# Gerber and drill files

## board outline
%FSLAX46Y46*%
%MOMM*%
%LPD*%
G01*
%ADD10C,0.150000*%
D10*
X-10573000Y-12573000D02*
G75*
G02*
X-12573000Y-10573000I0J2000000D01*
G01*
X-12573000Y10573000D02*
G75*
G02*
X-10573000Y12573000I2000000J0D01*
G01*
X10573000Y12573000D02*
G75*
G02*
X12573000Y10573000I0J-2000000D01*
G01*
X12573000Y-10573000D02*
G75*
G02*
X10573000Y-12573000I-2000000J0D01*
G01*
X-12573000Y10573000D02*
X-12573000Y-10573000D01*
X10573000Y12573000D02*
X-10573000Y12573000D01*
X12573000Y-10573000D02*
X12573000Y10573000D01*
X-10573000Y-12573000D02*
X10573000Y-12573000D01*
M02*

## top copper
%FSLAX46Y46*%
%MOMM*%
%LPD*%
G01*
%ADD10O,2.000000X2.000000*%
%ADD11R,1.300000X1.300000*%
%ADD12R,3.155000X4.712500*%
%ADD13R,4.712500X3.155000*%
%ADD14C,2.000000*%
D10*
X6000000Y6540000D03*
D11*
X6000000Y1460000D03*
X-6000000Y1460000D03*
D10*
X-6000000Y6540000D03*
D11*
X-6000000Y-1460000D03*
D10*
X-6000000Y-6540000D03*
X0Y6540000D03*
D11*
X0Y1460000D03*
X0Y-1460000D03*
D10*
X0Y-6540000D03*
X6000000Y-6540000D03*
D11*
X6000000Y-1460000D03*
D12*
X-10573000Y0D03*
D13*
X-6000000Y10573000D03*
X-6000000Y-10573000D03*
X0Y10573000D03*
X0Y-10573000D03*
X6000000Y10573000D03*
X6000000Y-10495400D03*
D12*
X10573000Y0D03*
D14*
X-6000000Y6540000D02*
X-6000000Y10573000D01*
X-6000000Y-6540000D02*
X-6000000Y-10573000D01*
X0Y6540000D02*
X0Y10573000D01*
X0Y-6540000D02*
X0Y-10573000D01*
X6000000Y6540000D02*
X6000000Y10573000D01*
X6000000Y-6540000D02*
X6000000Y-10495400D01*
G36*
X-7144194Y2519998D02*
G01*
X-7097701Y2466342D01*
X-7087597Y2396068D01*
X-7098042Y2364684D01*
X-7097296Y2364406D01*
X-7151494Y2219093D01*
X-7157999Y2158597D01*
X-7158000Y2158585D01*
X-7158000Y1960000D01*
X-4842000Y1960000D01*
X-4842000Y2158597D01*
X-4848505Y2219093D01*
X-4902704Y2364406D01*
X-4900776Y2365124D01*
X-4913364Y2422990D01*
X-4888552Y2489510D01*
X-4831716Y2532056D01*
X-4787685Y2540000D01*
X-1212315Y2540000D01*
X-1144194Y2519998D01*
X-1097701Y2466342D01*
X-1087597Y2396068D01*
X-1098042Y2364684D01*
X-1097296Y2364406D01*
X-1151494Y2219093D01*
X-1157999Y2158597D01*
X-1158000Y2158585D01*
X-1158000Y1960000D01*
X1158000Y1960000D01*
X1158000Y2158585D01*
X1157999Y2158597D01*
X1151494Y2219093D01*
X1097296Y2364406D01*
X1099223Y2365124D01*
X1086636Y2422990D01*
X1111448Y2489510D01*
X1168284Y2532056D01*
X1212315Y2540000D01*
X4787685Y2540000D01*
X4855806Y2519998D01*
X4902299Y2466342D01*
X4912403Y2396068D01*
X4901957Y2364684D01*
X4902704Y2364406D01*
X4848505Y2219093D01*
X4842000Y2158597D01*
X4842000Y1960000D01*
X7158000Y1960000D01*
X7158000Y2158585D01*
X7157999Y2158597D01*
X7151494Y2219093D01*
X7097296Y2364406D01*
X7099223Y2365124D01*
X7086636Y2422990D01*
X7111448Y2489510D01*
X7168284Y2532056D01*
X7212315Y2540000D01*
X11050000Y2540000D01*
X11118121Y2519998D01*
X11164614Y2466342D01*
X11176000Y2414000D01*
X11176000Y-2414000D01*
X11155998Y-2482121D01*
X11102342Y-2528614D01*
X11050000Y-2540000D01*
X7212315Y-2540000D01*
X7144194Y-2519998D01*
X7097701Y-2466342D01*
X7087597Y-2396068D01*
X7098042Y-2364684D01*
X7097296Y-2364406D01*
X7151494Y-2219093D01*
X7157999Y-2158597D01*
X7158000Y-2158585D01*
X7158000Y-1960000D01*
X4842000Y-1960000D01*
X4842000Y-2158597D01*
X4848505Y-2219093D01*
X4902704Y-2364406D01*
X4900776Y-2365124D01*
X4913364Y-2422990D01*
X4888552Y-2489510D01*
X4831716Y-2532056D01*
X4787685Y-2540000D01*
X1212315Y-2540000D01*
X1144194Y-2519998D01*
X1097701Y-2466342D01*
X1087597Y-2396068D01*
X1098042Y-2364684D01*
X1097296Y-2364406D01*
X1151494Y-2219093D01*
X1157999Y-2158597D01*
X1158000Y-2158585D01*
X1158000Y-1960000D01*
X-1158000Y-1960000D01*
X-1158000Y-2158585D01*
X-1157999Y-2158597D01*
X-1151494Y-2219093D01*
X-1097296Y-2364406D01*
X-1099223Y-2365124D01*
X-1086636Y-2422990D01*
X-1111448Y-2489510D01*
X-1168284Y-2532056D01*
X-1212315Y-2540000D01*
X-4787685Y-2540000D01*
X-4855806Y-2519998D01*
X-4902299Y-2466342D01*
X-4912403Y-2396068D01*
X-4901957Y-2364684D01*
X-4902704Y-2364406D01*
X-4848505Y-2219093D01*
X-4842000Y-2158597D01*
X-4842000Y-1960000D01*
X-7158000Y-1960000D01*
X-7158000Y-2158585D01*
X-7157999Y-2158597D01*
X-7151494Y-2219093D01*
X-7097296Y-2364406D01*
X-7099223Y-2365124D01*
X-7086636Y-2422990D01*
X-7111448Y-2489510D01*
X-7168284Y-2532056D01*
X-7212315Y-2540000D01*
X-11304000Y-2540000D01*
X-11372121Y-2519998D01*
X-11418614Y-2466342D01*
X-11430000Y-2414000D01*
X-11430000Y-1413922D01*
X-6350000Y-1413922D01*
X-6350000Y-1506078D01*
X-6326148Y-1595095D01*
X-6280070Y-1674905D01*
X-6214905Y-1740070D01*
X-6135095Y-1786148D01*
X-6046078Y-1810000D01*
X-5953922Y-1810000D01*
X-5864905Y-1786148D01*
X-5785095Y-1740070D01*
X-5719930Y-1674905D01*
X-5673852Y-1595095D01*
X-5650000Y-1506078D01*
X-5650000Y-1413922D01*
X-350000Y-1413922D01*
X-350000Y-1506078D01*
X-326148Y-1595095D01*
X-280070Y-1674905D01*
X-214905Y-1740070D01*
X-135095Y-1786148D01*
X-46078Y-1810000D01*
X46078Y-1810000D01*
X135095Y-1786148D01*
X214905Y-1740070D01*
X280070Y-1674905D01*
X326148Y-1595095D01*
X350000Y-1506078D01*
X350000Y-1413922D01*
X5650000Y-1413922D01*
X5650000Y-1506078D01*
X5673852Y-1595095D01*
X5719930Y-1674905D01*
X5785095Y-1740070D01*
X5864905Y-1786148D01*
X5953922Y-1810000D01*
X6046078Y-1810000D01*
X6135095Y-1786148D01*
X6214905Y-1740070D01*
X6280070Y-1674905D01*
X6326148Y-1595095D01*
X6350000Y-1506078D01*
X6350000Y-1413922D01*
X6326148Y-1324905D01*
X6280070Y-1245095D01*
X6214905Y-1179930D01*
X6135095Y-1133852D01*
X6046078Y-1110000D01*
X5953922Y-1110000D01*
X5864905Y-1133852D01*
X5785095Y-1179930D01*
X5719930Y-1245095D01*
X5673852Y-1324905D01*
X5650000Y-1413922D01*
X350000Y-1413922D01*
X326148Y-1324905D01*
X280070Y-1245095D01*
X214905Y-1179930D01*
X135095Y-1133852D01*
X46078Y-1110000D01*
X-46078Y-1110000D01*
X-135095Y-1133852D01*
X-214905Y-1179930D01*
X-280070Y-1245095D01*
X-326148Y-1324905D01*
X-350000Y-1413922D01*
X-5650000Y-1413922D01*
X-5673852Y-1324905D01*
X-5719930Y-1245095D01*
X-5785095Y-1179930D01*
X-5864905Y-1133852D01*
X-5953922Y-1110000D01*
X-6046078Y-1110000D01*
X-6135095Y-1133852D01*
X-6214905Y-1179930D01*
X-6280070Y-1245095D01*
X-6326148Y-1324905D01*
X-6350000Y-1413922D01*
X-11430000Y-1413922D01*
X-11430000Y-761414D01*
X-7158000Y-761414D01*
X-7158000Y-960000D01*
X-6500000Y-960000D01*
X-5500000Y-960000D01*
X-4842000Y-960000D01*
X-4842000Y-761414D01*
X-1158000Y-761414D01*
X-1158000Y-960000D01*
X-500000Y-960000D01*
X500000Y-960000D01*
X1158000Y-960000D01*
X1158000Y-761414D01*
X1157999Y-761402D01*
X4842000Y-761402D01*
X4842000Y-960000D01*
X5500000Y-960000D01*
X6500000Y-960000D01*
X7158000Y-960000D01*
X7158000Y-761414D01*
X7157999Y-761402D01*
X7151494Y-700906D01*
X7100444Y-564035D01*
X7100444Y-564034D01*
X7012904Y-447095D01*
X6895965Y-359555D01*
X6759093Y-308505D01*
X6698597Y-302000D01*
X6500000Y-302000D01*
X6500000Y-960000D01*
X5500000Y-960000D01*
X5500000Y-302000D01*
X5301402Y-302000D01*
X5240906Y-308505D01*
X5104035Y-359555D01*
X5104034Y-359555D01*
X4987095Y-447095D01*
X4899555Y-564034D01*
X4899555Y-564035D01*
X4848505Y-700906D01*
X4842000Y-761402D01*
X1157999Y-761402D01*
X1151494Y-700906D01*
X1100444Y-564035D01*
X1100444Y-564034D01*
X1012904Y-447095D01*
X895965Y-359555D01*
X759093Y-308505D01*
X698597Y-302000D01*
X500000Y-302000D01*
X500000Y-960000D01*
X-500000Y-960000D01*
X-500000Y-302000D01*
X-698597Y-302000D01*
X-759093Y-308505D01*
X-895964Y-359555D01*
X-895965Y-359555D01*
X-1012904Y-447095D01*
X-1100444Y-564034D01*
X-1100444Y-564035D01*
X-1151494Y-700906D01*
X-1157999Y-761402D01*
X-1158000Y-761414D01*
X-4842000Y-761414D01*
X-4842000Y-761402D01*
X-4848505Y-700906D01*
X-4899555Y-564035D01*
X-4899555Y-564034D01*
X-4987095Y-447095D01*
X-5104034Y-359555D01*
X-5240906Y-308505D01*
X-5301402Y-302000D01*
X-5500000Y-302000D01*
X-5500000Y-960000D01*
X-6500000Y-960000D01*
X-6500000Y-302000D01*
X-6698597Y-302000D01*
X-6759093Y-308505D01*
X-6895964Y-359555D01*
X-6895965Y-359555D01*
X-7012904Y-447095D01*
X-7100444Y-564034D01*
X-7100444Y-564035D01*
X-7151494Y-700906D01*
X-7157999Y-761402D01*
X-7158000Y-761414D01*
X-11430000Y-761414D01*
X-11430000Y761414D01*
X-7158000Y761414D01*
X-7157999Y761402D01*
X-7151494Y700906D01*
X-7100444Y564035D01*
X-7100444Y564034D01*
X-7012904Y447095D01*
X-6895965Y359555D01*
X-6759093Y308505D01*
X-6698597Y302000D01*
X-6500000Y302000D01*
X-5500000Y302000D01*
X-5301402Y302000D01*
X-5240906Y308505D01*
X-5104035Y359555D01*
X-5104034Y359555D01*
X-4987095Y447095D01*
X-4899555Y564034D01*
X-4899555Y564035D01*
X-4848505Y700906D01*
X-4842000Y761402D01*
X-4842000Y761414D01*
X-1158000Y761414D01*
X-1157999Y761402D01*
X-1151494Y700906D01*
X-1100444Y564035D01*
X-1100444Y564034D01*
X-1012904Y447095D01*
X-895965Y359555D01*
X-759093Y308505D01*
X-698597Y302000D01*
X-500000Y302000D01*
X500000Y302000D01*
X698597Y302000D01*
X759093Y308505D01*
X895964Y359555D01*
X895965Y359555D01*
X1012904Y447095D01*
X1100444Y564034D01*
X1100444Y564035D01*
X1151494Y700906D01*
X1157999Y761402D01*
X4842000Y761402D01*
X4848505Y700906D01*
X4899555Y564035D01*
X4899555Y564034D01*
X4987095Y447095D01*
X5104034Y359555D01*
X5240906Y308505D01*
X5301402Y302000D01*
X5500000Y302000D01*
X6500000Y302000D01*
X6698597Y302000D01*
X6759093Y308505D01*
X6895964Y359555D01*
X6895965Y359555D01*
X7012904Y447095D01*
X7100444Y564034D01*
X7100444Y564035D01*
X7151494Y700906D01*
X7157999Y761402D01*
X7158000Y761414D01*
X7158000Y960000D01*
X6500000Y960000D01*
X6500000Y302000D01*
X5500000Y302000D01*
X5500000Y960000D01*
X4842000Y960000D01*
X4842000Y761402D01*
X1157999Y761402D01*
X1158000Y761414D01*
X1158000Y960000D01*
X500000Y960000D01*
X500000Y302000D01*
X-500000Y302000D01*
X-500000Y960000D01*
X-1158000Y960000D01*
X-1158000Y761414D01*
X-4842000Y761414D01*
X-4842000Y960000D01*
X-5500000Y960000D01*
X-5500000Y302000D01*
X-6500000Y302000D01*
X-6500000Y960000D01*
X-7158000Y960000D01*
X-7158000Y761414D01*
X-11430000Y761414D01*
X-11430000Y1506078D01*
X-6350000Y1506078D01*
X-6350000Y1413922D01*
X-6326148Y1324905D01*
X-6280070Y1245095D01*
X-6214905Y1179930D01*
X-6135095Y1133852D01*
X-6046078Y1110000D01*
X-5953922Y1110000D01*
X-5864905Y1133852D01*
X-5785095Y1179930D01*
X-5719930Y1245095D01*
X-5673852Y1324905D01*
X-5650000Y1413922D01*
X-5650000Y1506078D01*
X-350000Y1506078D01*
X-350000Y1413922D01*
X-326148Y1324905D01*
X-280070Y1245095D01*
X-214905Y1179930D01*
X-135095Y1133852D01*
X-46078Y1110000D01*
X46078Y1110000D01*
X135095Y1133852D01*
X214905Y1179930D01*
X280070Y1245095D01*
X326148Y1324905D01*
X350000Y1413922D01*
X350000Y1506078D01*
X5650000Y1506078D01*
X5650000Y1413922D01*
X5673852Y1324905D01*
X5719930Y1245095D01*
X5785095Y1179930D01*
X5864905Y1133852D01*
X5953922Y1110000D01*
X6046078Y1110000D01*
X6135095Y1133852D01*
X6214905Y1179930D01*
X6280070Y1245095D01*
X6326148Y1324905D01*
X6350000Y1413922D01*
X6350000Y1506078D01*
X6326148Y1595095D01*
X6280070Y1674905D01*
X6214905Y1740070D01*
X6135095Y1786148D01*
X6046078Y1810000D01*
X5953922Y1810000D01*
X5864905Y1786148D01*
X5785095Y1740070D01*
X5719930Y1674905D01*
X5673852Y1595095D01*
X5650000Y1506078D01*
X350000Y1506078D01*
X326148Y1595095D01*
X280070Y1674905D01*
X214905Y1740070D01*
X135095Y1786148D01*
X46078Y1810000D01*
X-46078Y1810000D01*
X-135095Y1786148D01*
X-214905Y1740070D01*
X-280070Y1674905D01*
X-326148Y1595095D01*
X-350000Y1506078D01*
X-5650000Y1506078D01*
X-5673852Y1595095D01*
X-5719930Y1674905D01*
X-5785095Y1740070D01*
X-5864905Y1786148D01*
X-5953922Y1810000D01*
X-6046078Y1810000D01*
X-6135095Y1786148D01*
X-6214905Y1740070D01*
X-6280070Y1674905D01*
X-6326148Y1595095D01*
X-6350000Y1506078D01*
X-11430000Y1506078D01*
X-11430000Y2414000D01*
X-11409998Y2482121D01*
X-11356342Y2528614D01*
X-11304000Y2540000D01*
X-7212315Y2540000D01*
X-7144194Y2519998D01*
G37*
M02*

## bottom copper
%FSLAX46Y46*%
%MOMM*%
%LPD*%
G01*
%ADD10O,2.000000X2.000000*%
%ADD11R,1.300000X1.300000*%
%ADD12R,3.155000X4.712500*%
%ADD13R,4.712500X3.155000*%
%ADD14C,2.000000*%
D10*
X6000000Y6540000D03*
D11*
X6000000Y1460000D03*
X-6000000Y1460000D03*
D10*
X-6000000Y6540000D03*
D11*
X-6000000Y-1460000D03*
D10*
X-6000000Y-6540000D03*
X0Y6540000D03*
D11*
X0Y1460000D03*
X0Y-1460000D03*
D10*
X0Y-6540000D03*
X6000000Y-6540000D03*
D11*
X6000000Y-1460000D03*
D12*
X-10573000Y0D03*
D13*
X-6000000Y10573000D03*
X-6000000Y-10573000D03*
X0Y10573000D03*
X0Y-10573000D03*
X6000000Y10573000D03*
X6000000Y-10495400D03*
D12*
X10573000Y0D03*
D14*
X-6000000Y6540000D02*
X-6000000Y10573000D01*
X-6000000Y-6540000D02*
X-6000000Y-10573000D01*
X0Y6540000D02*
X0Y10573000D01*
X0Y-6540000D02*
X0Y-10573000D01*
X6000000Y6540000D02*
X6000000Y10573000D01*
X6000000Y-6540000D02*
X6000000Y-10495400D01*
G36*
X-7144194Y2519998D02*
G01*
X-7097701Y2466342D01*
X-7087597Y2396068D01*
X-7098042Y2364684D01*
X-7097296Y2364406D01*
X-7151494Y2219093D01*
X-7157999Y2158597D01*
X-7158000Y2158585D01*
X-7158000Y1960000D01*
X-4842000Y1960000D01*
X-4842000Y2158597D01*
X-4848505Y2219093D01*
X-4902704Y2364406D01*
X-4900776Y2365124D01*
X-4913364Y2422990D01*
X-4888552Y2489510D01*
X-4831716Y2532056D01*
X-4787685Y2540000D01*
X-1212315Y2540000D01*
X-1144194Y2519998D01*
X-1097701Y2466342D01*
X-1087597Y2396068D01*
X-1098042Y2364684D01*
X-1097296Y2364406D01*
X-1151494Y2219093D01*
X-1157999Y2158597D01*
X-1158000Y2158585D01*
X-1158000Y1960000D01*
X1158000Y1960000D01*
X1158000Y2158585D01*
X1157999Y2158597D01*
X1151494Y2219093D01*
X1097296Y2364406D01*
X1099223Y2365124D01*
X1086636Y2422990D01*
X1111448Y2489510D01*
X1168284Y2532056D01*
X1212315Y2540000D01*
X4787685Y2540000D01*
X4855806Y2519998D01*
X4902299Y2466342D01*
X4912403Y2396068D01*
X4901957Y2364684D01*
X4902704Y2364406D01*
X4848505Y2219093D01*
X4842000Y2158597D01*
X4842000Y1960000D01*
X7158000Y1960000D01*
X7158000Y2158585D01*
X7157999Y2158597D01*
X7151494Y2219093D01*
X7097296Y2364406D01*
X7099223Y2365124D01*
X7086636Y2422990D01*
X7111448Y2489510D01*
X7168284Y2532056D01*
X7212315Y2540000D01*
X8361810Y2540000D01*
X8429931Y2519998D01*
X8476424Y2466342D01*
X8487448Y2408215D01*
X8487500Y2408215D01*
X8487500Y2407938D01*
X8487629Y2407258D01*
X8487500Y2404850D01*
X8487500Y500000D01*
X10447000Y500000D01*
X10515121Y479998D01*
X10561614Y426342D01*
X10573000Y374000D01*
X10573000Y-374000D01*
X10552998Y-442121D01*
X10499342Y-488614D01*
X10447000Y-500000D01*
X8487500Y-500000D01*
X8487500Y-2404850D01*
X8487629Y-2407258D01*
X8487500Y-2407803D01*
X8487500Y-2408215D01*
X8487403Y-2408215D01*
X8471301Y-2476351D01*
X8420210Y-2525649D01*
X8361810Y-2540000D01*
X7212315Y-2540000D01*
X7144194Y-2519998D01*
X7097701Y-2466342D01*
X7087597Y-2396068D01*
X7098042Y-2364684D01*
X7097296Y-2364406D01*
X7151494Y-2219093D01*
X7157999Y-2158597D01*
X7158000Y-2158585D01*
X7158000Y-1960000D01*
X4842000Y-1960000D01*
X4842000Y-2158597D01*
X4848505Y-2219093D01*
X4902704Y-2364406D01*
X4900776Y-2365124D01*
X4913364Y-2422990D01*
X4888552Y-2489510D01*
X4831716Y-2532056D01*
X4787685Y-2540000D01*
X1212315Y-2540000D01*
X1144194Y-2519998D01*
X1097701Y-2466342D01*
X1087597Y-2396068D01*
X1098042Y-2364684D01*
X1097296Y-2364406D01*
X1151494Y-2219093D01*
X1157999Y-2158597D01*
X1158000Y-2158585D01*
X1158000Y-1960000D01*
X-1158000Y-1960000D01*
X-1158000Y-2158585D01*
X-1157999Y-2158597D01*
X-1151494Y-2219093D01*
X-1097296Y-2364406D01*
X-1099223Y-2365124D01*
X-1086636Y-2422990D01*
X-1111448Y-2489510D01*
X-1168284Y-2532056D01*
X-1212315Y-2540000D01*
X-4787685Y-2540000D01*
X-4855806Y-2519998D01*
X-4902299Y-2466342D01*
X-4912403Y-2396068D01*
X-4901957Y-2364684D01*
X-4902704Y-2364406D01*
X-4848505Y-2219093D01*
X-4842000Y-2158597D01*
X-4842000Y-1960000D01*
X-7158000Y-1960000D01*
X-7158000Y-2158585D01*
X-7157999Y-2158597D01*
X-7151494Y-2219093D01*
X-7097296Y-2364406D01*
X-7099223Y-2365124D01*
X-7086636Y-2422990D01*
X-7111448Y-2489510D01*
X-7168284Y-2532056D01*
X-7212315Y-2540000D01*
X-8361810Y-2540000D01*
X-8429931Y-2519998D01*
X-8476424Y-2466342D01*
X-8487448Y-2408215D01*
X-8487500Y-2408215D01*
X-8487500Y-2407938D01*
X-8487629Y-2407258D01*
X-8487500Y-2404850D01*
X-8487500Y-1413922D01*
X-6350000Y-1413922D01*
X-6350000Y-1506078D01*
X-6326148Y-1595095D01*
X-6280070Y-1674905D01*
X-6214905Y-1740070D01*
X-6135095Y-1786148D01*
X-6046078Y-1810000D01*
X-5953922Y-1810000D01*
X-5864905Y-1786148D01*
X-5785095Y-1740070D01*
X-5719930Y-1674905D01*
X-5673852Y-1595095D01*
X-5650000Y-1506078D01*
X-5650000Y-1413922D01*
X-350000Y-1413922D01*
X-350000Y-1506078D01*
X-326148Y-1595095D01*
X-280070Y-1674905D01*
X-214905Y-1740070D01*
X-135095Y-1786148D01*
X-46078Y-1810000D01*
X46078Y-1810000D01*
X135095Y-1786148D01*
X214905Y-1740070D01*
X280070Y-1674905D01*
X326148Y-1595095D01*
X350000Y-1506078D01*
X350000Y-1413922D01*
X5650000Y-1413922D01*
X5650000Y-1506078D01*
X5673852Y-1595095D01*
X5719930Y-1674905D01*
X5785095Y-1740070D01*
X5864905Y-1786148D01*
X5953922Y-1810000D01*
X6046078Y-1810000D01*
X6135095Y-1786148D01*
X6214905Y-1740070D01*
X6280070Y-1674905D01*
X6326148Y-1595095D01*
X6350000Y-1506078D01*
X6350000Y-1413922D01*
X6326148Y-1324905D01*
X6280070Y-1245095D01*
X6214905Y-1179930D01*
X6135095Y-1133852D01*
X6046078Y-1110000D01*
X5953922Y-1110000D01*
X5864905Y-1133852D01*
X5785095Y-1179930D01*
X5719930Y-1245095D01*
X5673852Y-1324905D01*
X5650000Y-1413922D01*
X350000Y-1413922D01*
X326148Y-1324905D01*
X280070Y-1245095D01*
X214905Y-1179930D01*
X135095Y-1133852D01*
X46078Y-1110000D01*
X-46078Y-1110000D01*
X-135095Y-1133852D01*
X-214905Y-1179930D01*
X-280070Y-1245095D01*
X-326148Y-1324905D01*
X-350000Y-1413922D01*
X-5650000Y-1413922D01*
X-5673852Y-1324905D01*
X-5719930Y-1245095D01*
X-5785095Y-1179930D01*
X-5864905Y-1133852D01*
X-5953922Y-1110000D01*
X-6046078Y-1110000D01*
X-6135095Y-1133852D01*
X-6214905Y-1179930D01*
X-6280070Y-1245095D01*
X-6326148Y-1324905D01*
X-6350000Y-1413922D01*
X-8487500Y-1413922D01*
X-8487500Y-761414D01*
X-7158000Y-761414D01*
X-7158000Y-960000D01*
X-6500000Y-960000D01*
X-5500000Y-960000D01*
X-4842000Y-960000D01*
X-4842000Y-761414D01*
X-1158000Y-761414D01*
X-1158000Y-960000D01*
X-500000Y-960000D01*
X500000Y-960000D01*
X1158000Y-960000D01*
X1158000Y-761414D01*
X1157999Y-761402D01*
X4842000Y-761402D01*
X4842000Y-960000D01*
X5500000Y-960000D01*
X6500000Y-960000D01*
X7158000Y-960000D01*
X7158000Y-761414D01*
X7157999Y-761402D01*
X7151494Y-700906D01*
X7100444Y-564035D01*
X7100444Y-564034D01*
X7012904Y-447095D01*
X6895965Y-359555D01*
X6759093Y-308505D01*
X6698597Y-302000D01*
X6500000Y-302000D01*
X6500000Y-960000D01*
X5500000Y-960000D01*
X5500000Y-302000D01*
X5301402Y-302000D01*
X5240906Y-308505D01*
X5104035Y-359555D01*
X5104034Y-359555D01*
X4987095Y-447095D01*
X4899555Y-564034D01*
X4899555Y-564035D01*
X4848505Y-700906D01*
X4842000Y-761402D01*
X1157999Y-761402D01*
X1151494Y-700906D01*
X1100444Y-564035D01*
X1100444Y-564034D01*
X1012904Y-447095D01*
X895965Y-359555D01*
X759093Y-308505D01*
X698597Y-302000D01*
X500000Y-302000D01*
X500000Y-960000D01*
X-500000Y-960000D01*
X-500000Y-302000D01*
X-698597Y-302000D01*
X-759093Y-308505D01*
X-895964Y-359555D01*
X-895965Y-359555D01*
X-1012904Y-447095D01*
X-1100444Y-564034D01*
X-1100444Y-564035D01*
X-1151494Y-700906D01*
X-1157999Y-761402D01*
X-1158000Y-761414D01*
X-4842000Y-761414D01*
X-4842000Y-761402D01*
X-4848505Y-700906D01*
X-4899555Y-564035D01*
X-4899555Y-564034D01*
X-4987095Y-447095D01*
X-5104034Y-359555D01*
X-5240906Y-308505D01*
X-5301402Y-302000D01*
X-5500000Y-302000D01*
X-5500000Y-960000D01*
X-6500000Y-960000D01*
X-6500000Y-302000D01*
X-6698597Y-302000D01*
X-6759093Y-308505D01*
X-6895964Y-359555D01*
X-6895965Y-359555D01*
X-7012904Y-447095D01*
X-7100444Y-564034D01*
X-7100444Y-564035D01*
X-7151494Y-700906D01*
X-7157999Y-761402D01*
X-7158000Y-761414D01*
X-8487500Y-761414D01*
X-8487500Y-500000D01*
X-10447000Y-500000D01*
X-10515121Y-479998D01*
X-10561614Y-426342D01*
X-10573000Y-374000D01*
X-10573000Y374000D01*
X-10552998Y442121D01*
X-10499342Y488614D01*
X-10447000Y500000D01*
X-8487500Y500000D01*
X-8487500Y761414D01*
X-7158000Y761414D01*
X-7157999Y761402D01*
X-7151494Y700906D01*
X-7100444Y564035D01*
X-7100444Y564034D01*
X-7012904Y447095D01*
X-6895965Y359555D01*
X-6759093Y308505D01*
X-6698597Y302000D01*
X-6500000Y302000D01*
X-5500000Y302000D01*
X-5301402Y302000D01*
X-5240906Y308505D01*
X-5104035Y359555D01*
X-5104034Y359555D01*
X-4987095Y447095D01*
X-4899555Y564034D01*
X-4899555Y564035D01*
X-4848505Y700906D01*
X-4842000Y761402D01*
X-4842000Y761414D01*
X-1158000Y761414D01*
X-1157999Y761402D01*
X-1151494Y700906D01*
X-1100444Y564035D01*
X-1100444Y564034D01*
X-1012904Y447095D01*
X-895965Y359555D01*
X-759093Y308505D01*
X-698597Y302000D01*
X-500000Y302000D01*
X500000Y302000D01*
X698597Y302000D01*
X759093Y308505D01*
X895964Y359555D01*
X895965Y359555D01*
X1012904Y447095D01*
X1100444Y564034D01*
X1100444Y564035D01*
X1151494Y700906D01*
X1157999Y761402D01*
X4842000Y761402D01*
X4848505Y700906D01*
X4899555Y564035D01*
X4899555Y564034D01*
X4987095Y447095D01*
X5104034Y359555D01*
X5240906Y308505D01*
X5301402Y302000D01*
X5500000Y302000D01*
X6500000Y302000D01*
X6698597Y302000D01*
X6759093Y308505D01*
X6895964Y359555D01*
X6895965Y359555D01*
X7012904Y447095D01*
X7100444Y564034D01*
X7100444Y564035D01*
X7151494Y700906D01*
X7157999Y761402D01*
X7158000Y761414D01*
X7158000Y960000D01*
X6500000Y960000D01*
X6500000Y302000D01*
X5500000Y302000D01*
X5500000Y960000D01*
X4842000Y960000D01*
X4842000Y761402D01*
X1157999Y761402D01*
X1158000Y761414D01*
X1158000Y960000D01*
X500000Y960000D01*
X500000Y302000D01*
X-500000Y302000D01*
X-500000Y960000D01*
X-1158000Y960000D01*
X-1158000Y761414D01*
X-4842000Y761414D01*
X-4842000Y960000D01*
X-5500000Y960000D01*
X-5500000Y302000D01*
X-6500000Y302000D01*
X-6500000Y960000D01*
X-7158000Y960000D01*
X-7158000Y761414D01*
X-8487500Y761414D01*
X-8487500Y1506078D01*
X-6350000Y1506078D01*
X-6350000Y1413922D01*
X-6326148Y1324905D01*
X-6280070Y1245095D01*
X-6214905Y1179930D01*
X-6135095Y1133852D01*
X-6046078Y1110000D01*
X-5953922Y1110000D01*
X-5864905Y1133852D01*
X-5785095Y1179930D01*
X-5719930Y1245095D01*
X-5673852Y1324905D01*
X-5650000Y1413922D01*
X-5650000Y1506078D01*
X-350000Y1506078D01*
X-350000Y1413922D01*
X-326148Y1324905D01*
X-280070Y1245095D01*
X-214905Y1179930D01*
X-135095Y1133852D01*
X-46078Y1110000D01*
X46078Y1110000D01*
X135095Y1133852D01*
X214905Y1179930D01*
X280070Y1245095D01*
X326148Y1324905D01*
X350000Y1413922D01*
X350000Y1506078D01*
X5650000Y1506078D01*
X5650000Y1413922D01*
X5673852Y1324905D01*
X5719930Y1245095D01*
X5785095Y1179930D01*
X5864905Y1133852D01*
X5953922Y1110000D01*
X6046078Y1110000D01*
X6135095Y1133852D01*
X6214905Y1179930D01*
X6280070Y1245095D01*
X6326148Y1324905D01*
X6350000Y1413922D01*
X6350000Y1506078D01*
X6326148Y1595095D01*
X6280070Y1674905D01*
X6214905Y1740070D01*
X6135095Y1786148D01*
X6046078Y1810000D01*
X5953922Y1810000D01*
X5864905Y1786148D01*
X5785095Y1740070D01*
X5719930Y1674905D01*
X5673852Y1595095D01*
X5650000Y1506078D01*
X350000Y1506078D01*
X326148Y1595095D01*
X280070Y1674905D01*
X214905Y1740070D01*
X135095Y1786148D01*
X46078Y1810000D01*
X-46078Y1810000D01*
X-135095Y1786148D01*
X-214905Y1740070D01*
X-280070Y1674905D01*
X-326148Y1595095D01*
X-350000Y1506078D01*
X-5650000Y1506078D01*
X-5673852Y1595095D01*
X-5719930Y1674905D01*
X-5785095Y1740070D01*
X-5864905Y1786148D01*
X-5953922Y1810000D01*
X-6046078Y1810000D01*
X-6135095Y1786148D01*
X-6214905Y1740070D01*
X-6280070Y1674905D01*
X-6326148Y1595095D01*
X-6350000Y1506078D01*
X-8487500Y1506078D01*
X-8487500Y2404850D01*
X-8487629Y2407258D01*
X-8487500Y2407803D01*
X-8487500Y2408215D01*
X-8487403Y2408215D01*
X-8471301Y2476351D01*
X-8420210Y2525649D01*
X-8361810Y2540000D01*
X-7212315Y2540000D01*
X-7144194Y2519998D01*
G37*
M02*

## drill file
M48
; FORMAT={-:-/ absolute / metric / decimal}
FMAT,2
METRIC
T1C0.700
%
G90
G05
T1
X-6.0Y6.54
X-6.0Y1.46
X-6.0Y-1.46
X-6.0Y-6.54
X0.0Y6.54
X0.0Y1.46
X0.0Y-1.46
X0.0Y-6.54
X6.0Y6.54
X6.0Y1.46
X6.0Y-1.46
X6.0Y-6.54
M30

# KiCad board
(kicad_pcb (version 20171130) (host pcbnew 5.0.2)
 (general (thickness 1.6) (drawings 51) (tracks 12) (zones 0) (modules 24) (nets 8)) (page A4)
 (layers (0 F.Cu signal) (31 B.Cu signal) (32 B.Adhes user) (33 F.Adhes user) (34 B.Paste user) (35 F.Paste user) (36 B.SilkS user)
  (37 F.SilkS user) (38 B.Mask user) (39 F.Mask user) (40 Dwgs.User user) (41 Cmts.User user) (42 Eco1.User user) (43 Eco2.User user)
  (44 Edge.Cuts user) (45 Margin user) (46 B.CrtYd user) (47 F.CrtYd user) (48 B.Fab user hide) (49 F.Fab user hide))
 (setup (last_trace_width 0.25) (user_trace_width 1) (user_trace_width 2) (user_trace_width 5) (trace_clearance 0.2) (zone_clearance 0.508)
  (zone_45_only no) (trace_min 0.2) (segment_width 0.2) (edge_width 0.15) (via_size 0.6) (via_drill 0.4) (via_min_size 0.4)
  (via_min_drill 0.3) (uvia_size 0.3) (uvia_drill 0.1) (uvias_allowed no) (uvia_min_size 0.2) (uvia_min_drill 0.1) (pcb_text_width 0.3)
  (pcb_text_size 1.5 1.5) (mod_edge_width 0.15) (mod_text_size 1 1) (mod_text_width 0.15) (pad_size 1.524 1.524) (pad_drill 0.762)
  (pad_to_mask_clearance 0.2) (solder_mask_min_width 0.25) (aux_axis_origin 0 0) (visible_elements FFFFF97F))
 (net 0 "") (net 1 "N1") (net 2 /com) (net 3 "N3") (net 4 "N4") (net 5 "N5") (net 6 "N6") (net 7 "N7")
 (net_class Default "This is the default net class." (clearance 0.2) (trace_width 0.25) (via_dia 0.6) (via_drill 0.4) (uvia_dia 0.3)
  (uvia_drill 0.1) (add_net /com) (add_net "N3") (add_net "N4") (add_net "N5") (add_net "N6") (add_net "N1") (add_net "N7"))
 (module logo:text (layer F.Cu) (at 0.254 3.81)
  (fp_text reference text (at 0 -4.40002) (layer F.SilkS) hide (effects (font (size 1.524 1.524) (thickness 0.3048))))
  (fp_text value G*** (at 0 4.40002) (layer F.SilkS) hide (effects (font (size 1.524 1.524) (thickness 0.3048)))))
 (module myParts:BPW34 (layer B.Cu) (at 6 -1.46 90)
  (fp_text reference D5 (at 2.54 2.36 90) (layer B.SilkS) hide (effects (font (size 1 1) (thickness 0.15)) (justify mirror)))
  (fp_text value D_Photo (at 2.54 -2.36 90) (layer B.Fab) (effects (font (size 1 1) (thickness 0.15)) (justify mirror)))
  (pad 2 thru_hole oval (at 5.08 0 90) (size 2 2) (drill 0.7) (layers *.Cu *.Mask) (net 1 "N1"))
  (pad 1 thru_hole rect (at 0 0 90) (size 1.3 1.3) (drill 0.7) (layers *.Cu *.Mask) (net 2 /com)))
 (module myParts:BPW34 (layer B.Cu) (at -6 -1.46 90)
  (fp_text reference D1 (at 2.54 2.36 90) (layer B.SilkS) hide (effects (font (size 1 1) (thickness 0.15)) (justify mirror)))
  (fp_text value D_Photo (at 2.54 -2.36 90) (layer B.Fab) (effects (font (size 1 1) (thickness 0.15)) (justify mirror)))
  (pad 1 thru_hole rect (at 0 0 90) (size 1.3 1.3) (drill 0.7) (layers *.Cu *.Mask) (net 2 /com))
  (pad 2 thru_hole oval (at 5.08 0 90) (size 2 2) (drill 0.7) (layers *.Cu *.Mask) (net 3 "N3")))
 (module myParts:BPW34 (layer B.Cu) (at -6 1.46 270)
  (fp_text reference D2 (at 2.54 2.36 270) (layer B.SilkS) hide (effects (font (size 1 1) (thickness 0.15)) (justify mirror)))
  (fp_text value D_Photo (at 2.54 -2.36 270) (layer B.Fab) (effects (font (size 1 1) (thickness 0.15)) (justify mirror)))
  (pad 1 thru_hole rect (at 0 0 270) (size 1.3 1.3) (drill 0.7) (layers *.Cu *.Mask) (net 2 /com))
  (pad 2 thru_hole oval (at 5.08 0 270) (size 2 2) (drill 0.7) (layers *.Cu *.Mask) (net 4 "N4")))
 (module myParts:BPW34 (layer B.Cu) (at 0 -1.46 90)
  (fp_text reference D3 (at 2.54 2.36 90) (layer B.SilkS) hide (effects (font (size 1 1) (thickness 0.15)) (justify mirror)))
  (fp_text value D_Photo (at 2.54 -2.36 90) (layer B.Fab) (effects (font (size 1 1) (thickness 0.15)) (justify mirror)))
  (pad 2 thru_hole oval (at 5.08 0 90) (size 2 2) (drill 0.7) (layers *.Cu *.Mask) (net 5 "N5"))
  (pad 1 thru_hole rect (at 0 0 90) (size 1.3 1.3) (drill 0.7) (layers *.Cu *.Mask) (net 2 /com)))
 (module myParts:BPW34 (layer B.Cu) (at 0 1.46 270)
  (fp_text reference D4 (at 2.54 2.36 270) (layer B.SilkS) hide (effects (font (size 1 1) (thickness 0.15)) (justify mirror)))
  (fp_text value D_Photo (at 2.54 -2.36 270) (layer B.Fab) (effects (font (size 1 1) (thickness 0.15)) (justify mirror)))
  (pad 1 thru_hole rect (at 0 0 270) (size 1.3 1.3) (drill 0.7) (layers *.Cu *.Mask) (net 2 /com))
  (pad 2 thru_hole oval (at 5.08 0 270) (size 2 2) (drill 0.7) (layers *.Cu *.Mask) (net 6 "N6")))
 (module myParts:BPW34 (layer B.Cu) (at 6 1.46 270)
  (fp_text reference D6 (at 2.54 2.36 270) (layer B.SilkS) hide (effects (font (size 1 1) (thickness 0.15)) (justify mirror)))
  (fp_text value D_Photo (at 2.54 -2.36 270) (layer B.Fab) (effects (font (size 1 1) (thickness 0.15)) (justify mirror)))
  (pad 2 thru_hole oval (at 5.08 0 270) (size 2 2) (drill 0.7) (layers *.Cu *.Mask) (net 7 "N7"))
  (pad 1 thru_hole rect (at 0 0 270) (size 1.3 1.3) (drill 0.7) (layers *.Cu *.Mask) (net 2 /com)))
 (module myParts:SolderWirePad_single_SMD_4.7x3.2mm (layer F.Cu) (at -10.573 0 90)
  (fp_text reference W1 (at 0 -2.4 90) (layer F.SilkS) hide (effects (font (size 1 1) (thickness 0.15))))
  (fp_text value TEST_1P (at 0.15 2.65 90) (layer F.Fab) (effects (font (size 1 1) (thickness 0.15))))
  (pad 1 smd rect (at 0 0 90) (size 4.7125 3.155) (layers F.Cu F.Paste F.Mask) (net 2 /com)))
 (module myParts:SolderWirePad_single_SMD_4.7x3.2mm (layer F.Cu) (at -6 -10.573)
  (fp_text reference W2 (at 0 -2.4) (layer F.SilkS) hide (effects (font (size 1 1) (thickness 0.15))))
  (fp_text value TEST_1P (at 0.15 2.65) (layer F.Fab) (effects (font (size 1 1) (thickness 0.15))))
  (pad 1 smd rect (at 0 0) (size 4.7125 3.155) (layers F.Cu F.Paste F.Mask) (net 3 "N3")))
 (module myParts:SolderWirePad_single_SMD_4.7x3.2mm (layer F.Cu) (at -6 10.573)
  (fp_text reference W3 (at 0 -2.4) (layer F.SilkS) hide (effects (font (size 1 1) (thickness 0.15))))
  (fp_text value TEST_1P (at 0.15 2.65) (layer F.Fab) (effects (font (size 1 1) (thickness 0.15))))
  (pad 1 smd rect (at 0 0) (size 4.7125 3.155) (layers F.Cu F.Paste F.Mask) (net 4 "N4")))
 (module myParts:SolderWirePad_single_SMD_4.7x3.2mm (layer F.Cu) (at 0 -10.573)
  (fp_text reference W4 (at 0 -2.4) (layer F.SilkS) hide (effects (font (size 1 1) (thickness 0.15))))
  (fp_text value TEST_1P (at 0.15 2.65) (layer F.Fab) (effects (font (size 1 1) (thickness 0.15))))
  (pad 1 smd rect (at 0 0) (size 4.7125 3.155) (layers F.Cu F.Paste F.Mask) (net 5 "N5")))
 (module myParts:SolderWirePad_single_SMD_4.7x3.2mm (layer F.Cu) (at 0 10.573)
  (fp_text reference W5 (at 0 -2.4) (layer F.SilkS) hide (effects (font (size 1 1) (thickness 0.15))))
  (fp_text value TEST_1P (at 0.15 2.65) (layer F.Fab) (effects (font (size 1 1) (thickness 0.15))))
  (pad 1 smd rect (at 0 0) (size 4.7125 3.155) (layers F.Cu F.Paste F.Mask) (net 6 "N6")))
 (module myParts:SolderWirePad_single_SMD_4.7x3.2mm (layer F.Cu) (at 6 -10.573)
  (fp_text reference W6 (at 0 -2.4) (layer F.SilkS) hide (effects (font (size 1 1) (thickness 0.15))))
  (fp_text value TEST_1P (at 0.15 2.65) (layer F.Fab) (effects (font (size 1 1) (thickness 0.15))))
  (pad 1 smd rect (at 0 0) (size 4.7125 3.155) (layers F.Cu F.Paste F.Mask) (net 1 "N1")))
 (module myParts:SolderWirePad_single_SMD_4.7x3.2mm (layer F.Cu) (at 6 10.4954)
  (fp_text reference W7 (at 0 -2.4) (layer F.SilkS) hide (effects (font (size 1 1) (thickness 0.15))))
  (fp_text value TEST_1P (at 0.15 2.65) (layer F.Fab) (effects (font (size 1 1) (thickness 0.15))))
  (pad 1 smd rect (at 0 0) (size 4.7125 3.155) (layers F.Cu F.Paste F.Mask) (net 7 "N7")))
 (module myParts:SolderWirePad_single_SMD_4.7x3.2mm (layer F.Cu) (at 10.573 0 90)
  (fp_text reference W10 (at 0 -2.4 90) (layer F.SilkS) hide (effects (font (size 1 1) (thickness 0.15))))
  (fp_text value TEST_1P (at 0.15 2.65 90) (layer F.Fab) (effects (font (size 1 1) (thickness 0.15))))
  (pad 1 smd rect (at 0 0 90) (size 4.7125 3.155) (layers F.Cu F.Paste F.Mask) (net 2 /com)))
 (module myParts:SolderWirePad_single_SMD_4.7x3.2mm (layer B.Cu) (at -10.573 0 270)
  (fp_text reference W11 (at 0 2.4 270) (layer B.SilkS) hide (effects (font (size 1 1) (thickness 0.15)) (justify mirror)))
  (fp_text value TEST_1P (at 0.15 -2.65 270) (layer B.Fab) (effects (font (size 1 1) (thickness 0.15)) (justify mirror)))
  (pad 1 smd rect (at 0 0 270) (size 4.7125 3.155) (layers B.Cu B.Paste B.Mask) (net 2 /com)))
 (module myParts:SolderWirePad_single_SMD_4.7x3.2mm (layer B.Cu) (at -6 -10.573)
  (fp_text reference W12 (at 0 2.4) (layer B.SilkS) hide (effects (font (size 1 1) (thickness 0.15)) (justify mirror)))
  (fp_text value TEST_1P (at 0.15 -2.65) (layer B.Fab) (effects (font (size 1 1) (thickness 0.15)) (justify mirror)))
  (pad 1 smd rect (at 0 0) (size 4.7125 3.155) (layers B.Cu B.Paste B.Mask) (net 3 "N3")))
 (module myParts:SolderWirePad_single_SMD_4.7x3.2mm (layer B.Cu) (at -6 10.573)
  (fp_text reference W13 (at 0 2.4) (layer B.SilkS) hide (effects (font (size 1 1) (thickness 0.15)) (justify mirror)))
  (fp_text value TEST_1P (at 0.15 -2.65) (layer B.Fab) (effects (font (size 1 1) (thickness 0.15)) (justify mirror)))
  (pad 1 smd rect (at 0 0) (size 4.7125 3.155) (layers B.Cu B.Paste B.Mask) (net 4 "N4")))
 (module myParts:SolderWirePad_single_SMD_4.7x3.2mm (layer B.Cu) (at 0 -10.573)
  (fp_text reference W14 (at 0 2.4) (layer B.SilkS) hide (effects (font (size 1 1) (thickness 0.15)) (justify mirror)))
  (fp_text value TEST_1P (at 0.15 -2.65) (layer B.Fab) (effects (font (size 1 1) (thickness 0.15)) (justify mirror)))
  (pad 1 smd rect (at 0 0) (size 4.7125 3.155) (layers B.Cu B.Paste B.Mask) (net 5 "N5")))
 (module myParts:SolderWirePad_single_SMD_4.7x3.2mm (layer B.Cu) (at 0 10.573)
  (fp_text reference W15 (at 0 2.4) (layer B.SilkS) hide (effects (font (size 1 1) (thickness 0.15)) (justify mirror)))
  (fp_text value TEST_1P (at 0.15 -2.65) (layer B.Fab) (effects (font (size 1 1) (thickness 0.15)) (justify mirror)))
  (pad 1 smd rect (at 0 0) (size 4.7125 3.155) (layers B.Cu B.Paste B.Mask) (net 6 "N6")))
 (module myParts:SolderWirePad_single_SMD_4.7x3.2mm (layer B.Cu) (at 6 -10.573)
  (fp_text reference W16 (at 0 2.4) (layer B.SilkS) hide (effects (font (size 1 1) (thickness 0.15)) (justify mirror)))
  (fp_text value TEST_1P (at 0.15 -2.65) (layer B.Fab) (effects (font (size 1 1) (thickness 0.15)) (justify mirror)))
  (pad 1 smd rect (at 0 0) (size 4.7125 3.155) (layers B.Cu B.Paste B.Mask) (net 1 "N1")))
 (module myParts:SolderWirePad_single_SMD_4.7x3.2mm (layer B.Cu) (at 6 10.4954)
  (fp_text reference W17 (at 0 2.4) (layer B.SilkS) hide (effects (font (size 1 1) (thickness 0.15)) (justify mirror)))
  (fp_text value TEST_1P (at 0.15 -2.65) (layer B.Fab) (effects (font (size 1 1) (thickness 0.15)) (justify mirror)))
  (pad 1 smd rect (at 0 0) (size 4.7125 3.155) (layers B.Cu B.Paste B.Mask) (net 7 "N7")))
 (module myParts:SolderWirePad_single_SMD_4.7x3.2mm (layer B.Cu) (at 10.573 0 270)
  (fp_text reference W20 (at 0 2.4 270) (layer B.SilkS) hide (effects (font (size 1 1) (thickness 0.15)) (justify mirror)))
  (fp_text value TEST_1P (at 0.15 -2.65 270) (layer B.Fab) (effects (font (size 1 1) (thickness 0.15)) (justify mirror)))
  (pad 1 smd rect (at 0 0 270) (size 4.7125 3.155) (layers B.Cu B.Paste B.Mask) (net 2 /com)))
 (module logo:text (layer B.Cu) (at 0.254 4.064)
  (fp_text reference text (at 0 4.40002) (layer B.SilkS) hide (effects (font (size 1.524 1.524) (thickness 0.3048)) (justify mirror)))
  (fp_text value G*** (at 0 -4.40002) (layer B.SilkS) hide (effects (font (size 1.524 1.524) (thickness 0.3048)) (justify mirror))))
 (gr_arc (start -10.573 10.573) (end -10.573 12.573) (angle 90) (layer Edge.Cuts) (width 0.15))
 (gr_arc (start -10.573 -10.573) (end -12.573 -10.573) (angle 90) (layer Edge.Cuts) (width 0.15))
 (gr_arc (start 10.573 -10.573) (end 10.573 -12.573) (angle 90) (layer Edge.Cuts) (width 0.15))
 (gr_arc (start 10.573 10.573) (end 12.573 10.573) (angle 90) (layer Edge.Cuts) (width 0.15))
 (gr_line (start -12.573 -10.573) (end -12.573 10.573) (layer Edge.Cuts) (width 0.15))
 (gr_line (start 10.573 -12.573) (end -10.573 -12.573) (layer Edge.Cuts) (width 0.15))
 (gr_line (start 12.573 10.573) (end 12.573 -10.573) (layer Edge.Cuts) (width 0.15))
 (gr_line (start -10.573 12.573) (end 10.573 12.573) (layer Edge.Cuts) (width 0.15))
 (segment (start -6 -6.54) (end -6 -10.573) (width 2) (layer F.Cu) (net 3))
 (segment (start -6 -6.54) (end -6 -10.573) (width 2) (layer B.Cu) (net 3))
 (segment (start -6 6.54) (end -6 10.573) (width 2) (layer F.Cu) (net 4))
 (segment (start -6 6.54) (end -6 10.573) (width 2) (layer B.Cu) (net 4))
 (segment (start 0 -6.54) (end 0 -10.573) (width 2) (layer F.Cu) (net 5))
 (segment (start 0 -6.54) (end 0 -10.573) (width 2) (layer B.Cu) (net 5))
 (segment (start 0 6.54) (end 0 10.573) (width 2) (layer F.Cu) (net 6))
 (segment (start 0 6.54) (end 0 10.573) (width 2) (layer B.Cu) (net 6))
 (segment (start 6 -6.54) (end 6 -10.573) (width 2) (layer F.Cu) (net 1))
 (segment (start 6 -6.54) (end 6 -10.573) (width 2) (layer B.Cu) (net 1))
 (segment (start 6 6.54) (end 6 10.4954) (width 2) (layer F.Cu) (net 7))
 (segment (start 6 6.54) (end 6 10.4954) (width 2) (layer B.Cu) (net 7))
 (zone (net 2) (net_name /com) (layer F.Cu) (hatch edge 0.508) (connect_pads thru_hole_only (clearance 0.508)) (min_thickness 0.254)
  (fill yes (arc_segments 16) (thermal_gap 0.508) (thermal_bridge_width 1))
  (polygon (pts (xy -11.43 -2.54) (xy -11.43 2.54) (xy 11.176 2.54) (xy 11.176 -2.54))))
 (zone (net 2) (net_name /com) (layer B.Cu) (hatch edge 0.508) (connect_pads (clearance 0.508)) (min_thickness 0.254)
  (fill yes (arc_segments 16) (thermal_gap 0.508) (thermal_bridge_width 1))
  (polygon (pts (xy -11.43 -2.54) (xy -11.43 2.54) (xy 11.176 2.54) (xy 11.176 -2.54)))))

